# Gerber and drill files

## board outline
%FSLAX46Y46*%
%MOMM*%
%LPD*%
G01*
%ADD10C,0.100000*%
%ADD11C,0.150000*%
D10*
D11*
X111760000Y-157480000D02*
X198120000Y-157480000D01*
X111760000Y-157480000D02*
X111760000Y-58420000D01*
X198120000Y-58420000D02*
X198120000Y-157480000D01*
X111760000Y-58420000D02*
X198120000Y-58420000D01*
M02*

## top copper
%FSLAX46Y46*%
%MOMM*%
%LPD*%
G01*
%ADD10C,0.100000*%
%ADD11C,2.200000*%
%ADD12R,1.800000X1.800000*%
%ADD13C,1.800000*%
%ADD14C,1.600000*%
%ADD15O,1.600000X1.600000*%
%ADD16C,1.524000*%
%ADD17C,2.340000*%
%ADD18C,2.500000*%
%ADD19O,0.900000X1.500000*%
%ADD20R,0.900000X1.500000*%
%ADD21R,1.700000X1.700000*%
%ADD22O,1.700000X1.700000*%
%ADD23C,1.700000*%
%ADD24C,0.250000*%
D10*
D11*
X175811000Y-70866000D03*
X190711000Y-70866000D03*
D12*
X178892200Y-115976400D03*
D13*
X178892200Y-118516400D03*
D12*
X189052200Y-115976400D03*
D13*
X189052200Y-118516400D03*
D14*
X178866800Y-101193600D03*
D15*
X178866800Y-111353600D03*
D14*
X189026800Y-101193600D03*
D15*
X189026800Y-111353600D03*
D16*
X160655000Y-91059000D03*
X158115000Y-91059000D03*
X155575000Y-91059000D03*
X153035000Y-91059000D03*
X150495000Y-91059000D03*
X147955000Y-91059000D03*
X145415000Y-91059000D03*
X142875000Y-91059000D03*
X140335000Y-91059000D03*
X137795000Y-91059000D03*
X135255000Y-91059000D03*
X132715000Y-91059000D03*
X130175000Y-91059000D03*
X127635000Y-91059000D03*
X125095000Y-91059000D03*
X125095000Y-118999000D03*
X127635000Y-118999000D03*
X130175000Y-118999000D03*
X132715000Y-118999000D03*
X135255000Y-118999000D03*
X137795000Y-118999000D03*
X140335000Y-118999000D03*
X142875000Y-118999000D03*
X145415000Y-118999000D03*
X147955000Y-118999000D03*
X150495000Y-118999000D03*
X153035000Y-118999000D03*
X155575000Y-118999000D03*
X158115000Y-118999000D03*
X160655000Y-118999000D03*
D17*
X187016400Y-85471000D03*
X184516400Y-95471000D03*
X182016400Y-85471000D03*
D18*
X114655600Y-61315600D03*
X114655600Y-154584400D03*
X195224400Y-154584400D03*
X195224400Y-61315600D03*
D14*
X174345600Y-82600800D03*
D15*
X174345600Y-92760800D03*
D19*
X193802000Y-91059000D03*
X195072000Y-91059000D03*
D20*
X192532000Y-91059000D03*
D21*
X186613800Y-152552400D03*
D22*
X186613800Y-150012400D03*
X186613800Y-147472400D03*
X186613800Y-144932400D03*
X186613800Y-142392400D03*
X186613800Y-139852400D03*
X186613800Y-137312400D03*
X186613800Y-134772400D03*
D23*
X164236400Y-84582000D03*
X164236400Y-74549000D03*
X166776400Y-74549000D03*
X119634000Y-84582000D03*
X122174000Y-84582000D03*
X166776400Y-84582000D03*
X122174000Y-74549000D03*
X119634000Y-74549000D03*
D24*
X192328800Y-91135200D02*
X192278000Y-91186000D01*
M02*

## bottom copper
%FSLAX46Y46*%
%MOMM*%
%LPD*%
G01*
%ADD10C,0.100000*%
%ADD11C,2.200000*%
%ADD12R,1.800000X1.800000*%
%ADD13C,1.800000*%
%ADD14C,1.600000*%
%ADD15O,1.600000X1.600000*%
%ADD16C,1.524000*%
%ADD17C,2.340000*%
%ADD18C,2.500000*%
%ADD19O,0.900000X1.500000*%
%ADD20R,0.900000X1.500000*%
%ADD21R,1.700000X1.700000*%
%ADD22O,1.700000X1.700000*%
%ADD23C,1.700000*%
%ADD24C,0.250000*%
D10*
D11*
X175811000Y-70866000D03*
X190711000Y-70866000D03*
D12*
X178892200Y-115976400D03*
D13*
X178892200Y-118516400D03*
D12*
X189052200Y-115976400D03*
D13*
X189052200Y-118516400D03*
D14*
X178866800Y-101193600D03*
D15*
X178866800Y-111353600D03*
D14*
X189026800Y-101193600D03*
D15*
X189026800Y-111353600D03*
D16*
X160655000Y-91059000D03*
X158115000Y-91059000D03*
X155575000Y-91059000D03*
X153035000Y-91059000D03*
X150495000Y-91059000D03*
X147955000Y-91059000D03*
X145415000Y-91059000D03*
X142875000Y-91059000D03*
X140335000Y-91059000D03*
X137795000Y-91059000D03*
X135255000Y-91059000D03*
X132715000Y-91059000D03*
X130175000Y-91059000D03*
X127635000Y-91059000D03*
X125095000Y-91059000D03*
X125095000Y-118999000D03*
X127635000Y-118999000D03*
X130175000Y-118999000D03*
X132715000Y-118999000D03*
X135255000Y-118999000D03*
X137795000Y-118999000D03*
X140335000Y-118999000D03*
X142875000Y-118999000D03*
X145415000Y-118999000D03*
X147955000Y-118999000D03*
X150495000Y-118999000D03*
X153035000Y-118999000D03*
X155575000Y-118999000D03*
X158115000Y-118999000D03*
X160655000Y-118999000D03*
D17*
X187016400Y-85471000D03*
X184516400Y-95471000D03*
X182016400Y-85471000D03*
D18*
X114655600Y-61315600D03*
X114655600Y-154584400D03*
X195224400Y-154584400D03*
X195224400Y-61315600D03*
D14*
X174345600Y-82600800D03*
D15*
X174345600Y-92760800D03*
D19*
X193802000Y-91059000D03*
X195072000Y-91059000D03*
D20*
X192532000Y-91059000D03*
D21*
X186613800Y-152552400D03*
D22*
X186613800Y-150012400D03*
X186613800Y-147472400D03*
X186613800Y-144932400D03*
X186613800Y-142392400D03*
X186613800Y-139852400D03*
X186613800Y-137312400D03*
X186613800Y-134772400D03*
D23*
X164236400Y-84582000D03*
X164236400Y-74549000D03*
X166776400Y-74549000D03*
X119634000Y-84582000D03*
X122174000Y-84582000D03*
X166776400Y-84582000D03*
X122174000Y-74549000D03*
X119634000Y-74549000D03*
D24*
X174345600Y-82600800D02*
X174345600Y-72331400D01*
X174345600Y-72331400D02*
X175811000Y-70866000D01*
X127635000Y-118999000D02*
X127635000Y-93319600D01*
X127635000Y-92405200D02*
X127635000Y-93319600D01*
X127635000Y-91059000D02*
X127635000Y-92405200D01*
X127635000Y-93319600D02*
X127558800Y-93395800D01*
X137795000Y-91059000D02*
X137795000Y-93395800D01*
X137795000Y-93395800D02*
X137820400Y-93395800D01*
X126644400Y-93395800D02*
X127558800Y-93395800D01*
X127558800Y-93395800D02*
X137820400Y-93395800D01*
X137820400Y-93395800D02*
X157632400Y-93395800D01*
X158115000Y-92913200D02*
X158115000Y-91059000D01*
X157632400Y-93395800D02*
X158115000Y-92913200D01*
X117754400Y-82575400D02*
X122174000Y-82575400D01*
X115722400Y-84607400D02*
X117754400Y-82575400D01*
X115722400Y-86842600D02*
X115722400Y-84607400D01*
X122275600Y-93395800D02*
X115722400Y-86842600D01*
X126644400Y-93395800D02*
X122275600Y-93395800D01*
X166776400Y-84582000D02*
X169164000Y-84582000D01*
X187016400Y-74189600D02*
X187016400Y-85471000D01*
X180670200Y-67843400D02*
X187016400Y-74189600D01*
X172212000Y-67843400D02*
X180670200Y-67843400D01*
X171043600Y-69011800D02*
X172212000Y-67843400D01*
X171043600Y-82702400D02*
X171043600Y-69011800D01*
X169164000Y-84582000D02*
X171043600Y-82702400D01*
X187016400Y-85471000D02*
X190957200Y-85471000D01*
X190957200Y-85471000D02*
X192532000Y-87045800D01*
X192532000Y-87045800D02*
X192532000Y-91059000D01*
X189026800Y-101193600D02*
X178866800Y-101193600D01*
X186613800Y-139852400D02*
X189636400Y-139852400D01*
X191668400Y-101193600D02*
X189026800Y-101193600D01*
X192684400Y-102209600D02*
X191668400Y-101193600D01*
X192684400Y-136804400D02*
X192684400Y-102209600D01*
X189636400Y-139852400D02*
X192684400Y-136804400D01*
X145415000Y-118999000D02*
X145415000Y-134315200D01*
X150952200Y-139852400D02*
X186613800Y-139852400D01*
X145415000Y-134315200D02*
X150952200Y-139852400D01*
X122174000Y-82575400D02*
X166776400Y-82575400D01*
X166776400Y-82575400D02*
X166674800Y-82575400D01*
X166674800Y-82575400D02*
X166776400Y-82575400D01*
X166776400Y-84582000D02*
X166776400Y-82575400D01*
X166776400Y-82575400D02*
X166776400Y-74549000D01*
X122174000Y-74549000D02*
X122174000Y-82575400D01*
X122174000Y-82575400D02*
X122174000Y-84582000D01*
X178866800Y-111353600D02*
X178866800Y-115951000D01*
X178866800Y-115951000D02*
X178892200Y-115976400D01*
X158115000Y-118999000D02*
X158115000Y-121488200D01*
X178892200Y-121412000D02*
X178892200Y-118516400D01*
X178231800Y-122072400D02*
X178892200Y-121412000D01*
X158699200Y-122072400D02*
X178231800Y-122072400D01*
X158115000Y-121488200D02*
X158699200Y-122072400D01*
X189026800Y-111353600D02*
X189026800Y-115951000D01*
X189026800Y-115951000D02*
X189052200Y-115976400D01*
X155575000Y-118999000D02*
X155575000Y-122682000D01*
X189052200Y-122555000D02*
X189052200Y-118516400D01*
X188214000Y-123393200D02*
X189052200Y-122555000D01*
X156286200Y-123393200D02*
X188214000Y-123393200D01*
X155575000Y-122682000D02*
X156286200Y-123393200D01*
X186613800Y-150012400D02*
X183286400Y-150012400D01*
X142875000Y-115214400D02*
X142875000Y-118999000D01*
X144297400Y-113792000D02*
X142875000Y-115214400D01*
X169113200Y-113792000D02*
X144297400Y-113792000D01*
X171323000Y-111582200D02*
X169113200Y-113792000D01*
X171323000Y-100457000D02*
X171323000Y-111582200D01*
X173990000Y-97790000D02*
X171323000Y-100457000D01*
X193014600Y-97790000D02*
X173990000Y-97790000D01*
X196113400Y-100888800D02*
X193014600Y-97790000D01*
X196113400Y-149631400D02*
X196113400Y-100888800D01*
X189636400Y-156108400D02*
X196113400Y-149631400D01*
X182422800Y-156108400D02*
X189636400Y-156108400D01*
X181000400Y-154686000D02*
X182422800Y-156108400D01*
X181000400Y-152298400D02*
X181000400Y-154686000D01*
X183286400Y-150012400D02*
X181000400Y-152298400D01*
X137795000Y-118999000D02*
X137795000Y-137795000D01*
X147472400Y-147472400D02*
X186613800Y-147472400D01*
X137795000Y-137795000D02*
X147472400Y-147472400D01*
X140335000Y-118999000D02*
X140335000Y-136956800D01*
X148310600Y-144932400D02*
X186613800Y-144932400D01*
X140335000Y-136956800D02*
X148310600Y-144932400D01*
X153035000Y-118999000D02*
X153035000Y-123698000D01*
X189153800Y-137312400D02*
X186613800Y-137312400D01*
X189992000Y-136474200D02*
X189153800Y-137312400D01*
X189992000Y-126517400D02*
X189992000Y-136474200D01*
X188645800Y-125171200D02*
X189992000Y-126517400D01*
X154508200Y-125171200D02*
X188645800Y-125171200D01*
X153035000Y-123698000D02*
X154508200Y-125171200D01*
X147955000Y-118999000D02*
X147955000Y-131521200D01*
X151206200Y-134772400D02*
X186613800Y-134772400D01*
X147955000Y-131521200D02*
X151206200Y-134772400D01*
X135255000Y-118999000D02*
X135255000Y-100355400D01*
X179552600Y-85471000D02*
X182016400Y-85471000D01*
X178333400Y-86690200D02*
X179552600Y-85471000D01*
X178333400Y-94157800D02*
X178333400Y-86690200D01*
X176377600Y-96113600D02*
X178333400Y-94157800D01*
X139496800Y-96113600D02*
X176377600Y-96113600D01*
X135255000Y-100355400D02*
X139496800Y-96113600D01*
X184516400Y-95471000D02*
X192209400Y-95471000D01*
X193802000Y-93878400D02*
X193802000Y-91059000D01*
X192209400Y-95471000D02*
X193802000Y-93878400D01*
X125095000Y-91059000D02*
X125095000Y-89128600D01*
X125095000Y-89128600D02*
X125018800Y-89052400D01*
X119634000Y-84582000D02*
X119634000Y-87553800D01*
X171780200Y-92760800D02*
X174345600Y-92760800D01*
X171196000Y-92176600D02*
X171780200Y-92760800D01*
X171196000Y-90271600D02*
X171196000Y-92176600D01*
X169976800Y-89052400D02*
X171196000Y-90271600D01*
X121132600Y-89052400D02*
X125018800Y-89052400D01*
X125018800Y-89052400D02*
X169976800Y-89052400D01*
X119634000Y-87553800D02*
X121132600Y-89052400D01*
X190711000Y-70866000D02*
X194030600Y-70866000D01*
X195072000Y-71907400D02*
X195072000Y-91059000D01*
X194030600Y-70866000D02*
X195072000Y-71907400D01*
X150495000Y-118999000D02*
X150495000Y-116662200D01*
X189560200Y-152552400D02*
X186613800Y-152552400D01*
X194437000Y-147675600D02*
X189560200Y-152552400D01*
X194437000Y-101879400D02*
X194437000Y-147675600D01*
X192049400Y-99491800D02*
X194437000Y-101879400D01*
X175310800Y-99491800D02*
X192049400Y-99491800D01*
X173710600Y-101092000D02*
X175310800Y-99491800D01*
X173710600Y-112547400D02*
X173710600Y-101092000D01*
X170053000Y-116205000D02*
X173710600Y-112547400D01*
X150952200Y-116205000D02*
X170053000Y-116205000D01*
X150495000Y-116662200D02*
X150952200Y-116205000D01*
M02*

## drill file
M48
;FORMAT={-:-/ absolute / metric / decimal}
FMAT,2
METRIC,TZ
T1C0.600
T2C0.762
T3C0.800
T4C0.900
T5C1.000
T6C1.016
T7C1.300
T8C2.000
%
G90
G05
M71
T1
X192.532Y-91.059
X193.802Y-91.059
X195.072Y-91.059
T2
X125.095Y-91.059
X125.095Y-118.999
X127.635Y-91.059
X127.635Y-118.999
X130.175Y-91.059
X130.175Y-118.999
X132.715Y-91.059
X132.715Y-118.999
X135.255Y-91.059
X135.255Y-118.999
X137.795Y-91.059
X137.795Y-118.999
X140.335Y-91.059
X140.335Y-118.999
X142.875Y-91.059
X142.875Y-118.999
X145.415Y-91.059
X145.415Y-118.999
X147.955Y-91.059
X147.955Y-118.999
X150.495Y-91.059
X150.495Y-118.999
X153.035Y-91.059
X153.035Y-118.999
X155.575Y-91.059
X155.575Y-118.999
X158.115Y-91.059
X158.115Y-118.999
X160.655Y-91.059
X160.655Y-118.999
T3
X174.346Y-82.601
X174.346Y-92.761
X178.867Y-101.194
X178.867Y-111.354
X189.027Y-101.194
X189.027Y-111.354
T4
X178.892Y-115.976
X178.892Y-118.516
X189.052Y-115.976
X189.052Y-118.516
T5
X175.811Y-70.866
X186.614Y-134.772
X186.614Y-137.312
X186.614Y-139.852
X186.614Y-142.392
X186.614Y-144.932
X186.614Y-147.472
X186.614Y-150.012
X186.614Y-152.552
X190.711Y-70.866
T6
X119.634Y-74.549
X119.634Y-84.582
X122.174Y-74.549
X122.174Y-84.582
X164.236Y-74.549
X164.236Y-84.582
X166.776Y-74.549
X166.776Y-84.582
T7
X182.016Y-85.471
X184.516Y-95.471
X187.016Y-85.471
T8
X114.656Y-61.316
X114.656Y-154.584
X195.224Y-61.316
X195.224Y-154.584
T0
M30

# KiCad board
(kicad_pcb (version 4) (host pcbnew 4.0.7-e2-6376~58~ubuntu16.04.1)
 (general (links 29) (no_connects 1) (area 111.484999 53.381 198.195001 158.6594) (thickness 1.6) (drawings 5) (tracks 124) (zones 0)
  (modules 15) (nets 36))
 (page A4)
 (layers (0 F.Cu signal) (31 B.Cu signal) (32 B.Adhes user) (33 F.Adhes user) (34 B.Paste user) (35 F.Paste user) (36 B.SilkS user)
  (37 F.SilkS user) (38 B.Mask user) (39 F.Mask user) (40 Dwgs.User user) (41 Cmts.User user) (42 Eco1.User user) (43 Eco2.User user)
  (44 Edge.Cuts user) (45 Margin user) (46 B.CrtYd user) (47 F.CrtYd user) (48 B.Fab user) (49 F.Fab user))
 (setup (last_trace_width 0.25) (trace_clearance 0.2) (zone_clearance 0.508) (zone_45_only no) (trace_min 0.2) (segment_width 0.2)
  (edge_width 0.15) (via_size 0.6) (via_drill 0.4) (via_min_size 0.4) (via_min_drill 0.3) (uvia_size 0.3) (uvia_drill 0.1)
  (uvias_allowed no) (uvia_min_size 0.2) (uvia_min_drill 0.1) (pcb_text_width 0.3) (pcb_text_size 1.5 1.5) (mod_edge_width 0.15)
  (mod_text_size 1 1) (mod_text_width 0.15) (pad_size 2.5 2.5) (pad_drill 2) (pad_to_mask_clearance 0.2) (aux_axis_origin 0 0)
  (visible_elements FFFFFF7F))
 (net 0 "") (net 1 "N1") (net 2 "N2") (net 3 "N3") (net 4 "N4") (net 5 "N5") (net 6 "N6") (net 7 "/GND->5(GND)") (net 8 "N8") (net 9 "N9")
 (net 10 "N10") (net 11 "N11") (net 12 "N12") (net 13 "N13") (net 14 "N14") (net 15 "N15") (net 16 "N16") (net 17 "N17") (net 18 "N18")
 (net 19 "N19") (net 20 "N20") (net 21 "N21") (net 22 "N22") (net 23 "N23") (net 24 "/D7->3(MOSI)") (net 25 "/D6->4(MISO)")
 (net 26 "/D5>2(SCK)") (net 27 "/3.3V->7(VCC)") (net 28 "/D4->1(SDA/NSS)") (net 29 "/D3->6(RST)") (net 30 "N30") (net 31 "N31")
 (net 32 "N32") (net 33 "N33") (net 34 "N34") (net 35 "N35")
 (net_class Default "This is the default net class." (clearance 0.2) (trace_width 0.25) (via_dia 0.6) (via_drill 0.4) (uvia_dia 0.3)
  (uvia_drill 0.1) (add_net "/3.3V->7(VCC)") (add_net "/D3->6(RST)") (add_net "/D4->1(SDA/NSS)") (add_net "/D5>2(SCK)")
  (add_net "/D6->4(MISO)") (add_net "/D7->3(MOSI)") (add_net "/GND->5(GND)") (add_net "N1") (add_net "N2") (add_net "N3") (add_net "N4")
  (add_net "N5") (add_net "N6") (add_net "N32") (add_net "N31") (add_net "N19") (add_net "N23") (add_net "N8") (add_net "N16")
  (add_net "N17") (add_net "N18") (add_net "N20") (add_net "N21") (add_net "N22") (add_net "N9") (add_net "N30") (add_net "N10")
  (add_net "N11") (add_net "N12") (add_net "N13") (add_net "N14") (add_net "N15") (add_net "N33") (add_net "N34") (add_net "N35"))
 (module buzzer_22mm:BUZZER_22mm (layer F.Cu) (at 183.261 70.866)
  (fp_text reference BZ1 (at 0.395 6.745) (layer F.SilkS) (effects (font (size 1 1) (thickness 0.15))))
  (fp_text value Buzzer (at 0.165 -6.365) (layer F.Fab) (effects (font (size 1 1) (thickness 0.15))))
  (pad 1 thru_hole circle (at -7.45 0) (size 2.2 2.2) (drill 1) (layers *.Cu *.Mask) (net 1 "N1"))
  (pad 2 thru_hole circle (at 7.45 0) (size 2.2 2.2) (drill 1) (layers *.Cu *.Mask) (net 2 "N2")))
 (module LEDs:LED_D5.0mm (layer F.Cu) (at 178.8922 115.9764 270)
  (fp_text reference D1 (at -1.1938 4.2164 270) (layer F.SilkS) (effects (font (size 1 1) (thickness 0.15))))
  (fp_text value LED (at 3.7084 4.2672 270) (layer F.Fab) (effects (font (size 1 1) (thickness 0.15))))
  (pad 1 thru_hole rect (at 0 0 270) (size 1.8 1.8) (drill 0.9) (layers *.Cu *.Mask) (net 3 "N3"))
  (pad 2 thru_hole circle (at 2.54 0 270) (size 1.8 1.8) (drill 0.9) (layers *.Cu *.Mask) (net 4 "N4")))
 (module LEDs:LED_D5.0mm (layer F.Cu) (at 189.0522 115.9764 270)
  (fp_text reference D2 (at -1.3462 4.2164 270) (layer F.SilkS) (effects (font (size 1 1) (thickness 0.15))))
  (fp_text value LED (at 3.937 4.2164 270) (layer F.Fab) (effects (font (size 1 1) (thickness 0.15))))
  (pad 1 thru_hole rect (at 0 0 270) (size 1.8 1.8) (drill 0.9) (layers *.Cu *.Mask) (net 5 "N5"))
  (pad 2 thru_hole circle (at 2.54 0 270) (size 1.8 1.8) (drill 0.9) (layers *.Cu *.Mask) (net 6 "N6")))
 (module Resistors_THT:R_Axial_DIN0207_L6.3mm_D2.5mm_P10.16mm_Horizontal (layer F.Cu) (at 178.8668 101.1936 270)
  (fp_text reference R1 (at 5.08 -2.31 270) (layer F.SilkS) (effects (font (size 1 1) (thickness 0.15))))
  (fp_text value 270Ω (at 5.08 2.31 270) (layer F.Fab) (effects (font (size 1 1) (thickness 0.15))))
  (pad 1 thru_hole circle (at 0 0 270) (size 1.6 1.6) (drill 0.8) (layers *.Cu *.Mask) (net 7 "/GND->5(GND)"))
  (pad 2 thru_hole oval (at 10.16 0 270) (size 1.6 1.6) (drill 0.8) (layers *.Cu *.Mask) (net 3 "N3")))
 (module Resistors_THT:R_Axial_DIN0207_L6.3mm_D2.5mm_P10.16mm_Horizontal (layer F.Cu) (at 189.0268 101.1936 270)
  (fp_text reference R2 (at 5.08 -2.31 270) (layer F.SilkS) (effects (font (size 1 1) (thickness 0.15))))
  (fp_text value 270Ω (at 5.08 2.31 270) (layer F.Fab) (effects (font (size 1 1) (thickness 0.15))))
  (pad 1 thru_hole circle (at 0 0 270) (size 1.6 1.6) (drill 0.8) (layers *.Cu *.Mask) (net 7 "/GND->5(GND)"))
  (pad 2 thru_hole oval (at 10.16 0 270) (size 1.6 1.6) (drill 0.8) (layers *.Cu *.Mask) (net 5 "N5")))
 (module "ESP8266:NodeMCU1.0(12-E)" (layer F.Cu) (at 139.7 105.029 270)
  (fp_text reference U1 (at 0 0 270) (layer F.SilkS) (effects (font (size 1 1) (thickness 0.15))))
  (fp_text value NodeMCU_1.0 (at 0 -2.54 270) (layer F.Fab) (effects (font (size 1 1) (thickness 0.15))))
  (pad 1 thru_hole circle (at -13.97 -20.955 270) (size 1.524 1.524) (drill 0.762) (layers *.Cu *.Mask F.SilkS) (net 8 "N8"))
  (pad 2 thru_hole circle (at -13.97 -18.415 270) (size 1.524 1.524) (drill 0.762) (layers *.Cu *.Mask F.SilkS) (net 7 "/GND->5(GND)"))
  (pad 3 thru_hole circle (at -13.97 -15.875 270) (size 1.524 1.524) (drill 0.762) (layers *.Cu *.Mask F.SilkS) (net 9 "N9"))
  (pad 4 thru_hole circle (at -13.97 -13.335 270) (size 1.524 1.524) (drill 0.762) (layers *.Cu *.Mask F.SilkS) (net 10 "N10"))
  (pad 5 thru_hole circle (at -13.97 -10.795 270) (size 1.524 1.524) (drill 0.762) (layers *.Cu *.Mask F.SilkS) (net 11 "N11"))
  (pad 6 thru_hole circle (at -13.97 -8.255 270) (size 1.524 1.524) (drill 0.762) (layers *.Cu *.Mask F.SilkS) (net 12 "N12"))
  (pad 7 thru_hole circle (at -13.97 -5.715 270) (size 1.524 1.524) (drill 0.762) (layers *.Cu *.Mask F.SilkS) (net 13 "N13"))
  (pad 8 thru_hole circle (at -13.97 -3.175 270) (size 1.524 1.524) (drill 0.762) (layers *.Cu *.Mask F.SilkS) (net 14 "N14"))
  (pad 9 thru_hole circle (at -13.97 -0.635 270) (size 1.524 1.524) (drill 0.762) (layers *.Cu *.Mask F.SilkS) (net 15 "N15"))
  (pad 10 thru_hole circle (at -13.97 1.905 270) (size 1.524 1.524) (drill 0.762) (layers *.Cu *.Mask F.SilkS) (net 7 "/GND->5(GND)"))
  (pad 11 thru_hole circle (at -13.97 4.445 270) (size 1.524 1.524) (drill 0.762) (layers *.Cu *.Mask F.SilkS) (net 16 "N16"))
  (pad 12 thru_hole circle (at -13.97 6.985 270) (size 1.524 1.524) (drill 0.762) (layers *.Cu *.Mask F.SilkS) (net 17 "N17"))
  (pad 13 thru_hole circle (at -13.97 9.525 270) (size 1.524 1.524) (drill 0.762) (layers *.Cu *.Mask F.SilkS) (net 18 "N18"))
  (pad 14 thru_hole circle (at -13.97 12.065 270) (size 1.524 1.524) (drill 0.762) (layers *.Cu *.Mask F.SilkS) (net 7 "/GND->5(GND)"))
  (pad 15 thru_hole circle (at -13.97 14.605 270) (size 1.524 1.524) (drill 0.762) (layers *.Cu *.Mask F.SilkS) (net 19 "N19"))
  (pad 16 thru_hole circle (at 13.97 14.605 270) (size 1.524 1.524) (drill 0.762) (layers *.Cu *.Mask F.SilkS) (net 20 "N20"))
  (pad 17 thru_hole circle (at 13.97 12.065 270) (size 1.524 1.524) (drill 0.762) (layers *.Cu *.Mask F.SilkS) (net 7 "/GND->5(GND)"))
  (pad 18 thru_hole circle (at 13.97 9.525 270) (size 1.524 1.524) (drill 0.762) (layers *.Cu *.Mask F.SilkS) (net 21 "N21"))
  (pad 19 thru_hole circle (at 13.97 6.985 270) (size 1.524 1.524) (drill 0.762) (layers *.Cu *.Mask F.SilkS) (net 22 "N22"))
  (pad 20 thru_hole circle (at 13.97 4.445 270) (size 1.524 1.524) (drill 0.762) (layers *.Cu *.Mask F.SilkS) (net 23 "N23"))
  (pad 21 thru_hole circle (at 13.97 1.905 270) (size 1.524 1.524) (drill 0.762) (layers *.Cu *.Mask F.SilkS) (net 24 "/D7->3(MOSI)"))
  (pad 22 thru_hole circle (at 13.97 -0.635 270) (size 1.524 1.524) (drill 0.762) (layers *.Cu *.Mask F.SilkS) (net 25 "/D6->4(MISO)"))
  (pad 23 thru_hole circle (at 13.97 -3.175 270) (size 1.524 1.524) (drill 0.762) (layers *.Cu *.Mask F.SilkS) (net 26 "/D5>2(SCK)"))
  (pad 24 thru_hole circle (at 13.97 -5.715 270) (size 1.524 1.524) (drill 0.762) (layers *.Cu *.Mask F.SilkS) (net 7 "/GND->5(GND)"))
  (pad 25 thru_hole circle (at 13.97 -8.255 270) (size 1.524 1.524) (drill 0.762) (layers *.Cu *.Mask F.SilkS) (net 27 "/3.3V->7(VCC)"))
  (pad 26 thru_hole circle (at 13.97 -10.795 270) (size 1.524 1.524) (drill 0.762) (layers *.Cu *.Mask F.SilkS) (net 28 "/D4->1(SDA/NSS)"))
  (pad 27 thru_hole circle (at 13.97 -13.335 270) (size 1.524 1.524) (drill 0.762) (layers *.Cu *.Mask F.SilkS) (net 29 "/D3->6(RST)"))
  (pad 28 thru_hole circle (at 13.97 -15.875 270) (size 1.524 1.524) (drill 0.762) (layers *.Cu *.Mask F.SilkS) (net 6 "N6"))
  (pad 29 thru_hole circle (at 13.97 -18.415 270) (size 1.524 1.524) (drill 0.762) (layers *.Cu *.Mask F.SilkS) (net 4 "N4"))
  (pad 30 thru_hole circle (at 13.97 -20.955 270) (size 1.524 1.524) (drill 0.762) (layers *.Cu *.Mask F.SilkS) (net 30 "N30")))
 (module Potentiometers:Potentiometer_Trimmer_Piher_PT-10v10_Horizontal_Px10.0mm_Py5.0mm (layer F.Cu) (at 182.0164 85.471 270)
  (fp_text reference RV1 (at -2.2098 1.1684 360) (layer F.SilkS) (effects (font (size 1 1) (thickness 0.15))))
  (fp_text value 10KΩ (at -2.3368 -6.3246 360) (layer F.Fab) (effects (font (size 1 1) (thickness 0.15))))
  (pad 3 thru_hole circle (at 0 -5 270) (size 2.34 2.34) (drill 1.3) (layers *.Cu *.Mask) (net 7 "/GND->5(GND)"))
  (pad 2 thru_hole circle (at 10 -2.5 270) (size 2.34 2.34) (drill 1.3) (layers *.Cu *.Mask) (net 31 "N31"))
  (pad 1 thru_hole circle (at 0 0 270) (size 2.34 2.34) (drill 1.3) (layers *.Cu *.Mask) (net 23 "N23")))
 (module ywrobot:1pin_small (layer F.Cu) (at 114.6556 61.3156)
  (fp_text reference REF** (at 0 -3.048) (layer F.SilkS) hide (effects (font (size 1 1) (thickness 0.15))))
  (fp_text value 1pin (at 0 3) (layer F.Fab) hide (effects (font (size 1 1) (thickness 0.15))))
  (pad 1 thru_hole circle (at 0 0) (size 2.5 2.5) (drill 2) (layers *.Cu *.Mask) (zone_connect 0)))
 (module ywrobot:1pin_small (layer F.Cu) (at 114.6556 154.5844)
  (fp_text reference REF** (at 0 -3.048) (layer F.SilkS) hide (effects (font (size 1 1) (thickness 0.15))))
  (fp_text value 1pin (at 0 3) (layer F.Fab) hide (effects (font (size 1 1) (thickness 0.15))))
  (pad 2 thru_hole circle (at 0 0) (size 2.5 2.5) (drill 2) (layers *.Cu *.Mask) (zone_connect 0)))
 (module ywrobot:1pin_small (layer F.Cu) (at 195.2244 154.5844)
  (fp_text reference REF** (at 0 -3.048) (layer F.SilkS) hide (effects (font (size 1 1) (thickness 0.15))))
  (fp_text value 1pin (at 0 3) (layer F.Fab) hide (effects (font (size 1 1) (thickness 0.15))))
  (pad 3 thru_hole circle (at 0 0) (size 2.5 2.5) (drill 2) (layers *.Cu *.Mask) (zone_connect 0)))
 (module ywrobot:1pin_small (layer F.Cu) (at 195.2244 61.3156)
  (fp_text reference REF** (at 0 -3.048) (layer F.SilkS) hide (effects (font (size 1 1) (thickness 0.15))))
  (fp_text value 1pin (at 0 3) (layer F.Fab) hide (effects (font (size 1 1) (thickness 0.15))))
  (pad 4 thru_hole circle (at 0 0) (size 2.5 2.5) (drill 2) (layers *.Cu *.Mask) (zone_connect 0)))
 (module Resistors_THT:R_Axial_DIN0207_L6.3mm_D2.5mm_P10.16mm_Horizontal (layer F.Cu) (at 174.3456 82.6008 270)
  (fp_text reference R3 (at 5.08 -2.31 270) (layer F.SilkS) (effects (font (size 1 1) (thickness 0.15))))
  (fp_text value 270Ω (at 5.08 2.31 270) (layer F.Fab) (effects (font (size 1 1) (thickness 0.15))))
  (pad 1 thru_hole circle (at 0 0 270) (size 1.6 1.6) (drill 0.8) (layers *.Cu *.Mask) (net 1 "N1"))
  (pad 2 thru_hole oval (at 10.16 0 270) (size 1.6 1.6) (drill 0.8) (layers *.Cu *.Mask) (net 19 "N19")))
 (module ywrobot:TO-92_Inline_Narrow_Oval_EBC (layer F.Cu) (at 192.532 91.059)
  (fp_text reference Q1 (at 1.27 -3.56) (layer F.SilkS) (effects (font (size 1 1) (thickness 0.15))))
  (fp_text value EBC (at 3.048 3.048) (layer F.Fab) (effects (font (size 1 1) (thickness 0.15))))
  (pad 1 thru_hole oval (at 1.27 0 180) (size 0.9 1.5) (drill 0.6) (layers *.Cu *.Mask) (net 31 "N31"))
  (pad 2 thru_hole oval (at 2.54 0 180) (size 0.9 1.5) (drill 0.6) (layers *.Cu *.Mask) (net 2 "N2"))
  (pad 3 thru_hole rect (at 0 0 180) (size 0.9 1.5) (drill 0.6) (layers *.Cu *.Mask) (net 7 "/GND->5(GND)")))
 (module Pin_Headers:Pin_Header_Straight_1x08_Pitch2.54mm (layer F.Cu) (at 186.6138 152.5524 180)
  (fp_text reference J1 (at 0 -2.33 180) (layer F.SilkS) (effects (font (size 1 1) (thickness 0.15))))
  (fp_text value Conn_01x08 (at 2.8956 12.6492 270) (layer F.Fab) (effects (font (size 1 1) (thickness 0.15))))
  (pad 1 thru_hole rect (at 0 0 180) (size 1.7 1.7) (drill 1) (layers *.Cu *.Mask) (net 28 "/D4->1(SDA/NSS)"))
  (pad 2 thru_hole oval (at 0 2.54 180) (size 1.7 1.7) (drill 1) (layers *.Cu *.Mask) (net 26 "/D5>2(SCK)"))
  (pad 3 thru_hole oval (at 0 5.08 180) (size 1.7 1.7) (drill 1) (layers *.Cu *.Mask) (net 24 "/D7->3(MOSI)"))
  (pad 4 thru_hole oval (at 0 7.62 180) (size 1.7 1.7) (drill 1) (layers *.Cu *.Mask) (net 25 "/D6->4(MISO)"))
  (pad 5 thru_hole oval (at 0 10.16 180) (size 1.7 1.7) (drill 1) (layers *.Cu *.Mask) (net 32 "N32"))
  (pad 6 thru_hole oval (at 0 12.7 180) (size 1.7 1.7) (drill 1) (layers *.Cu *.Mask) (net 7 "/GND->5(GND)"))
  (pad 7 thru_hole oval (at 0 15.24 180) (size 1.7 1.7) (drill 1) (layers *.Cu *.Mask) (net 29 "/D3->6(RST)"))
  (pad 8 thru_hole oval (at 0 17.78 180) (size 1.7 1.7) (drill 1) (layers *.Cu *.Mask) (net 27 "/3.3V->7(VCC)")))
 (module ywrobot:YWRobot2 (layer F.Cu) (at 143.002 56.896 180)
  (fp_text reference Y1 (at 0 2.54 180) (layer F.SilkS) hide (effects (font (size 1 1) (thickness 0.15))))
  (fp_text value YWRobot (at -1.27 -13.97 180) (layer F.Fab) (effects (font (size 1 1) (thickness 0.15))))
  (pad 1 thru_hole circle (at -21.2344 -27.686 180) (size 1.7 1.7) (drill 1.016) (layers *.Cu *.Mask) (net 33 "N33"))
  (pad 2 thru_hole circle (at -21.2344 -17.653 180) (size 1.7 1.7) (drill 1.016) (layers *.Cu *.Mask) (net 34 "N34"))
  (pad 3 thru_hole circle (at -23.7744 -17.653 180) (size 1.7 1.7) (drill 1.016) (layers *.Cu *.Mask) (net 7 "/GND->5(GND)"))
  (pad 4 thru_hole circle (at 23.368 -27.686 180) (size 1.7 1.7) (drill 1.016) (layers *.Cu *.Mask) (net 19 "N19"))
  (pad 5 thru_hole circle (at 20.828 -27.686 180) (size 1.7 1.7) (drill 1.016) (layers *.Cu *.Mask) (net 7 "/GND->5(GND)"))
  (pad 6 thru_hole circle (at -23.7744 -27.686 180) (size 1.7 1.7) (drill 1.016) (layers *.Cu *.Mask) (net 7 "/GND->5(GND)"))
  (pad 7 thru_hole circle (at 20.828 -17.653 180) (size 1.7 1.7) (drill 1.016) (layers *.Cu *.Mask) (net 7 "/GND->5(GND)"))
  (pad 8 thru_hole circle (at 23.368 -17.653 180) (size 1.7 1.7) (drill 1.016) (layers *.Cu *.Mask) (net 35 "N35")))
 (gr_line (start 111.76 157.48) (end 198.12 157.48) (angle 90) (layer Edge.Cuts) (width 0.15))
 (gr_line (start 111.76 157.48) (end 111.76 58.42) (angle 90) (layer Edge.Cuts) (width 0.15))
 (gr_line (start 198.12 58.42) (end 198.12 157.48) (angle 90) (layer Edge.Cuts) (width 0.15))
 (gr_line (start 111.76 58.42) (end 198.12 58.42) (angle 90) (layer Edge.Cuts) (width 0.15))
 (segment (start 174.3456 82.6008) (end 174.3456 72.3314) (width 0.25) (layer B.Cu) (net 1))
 (segment (start 174.3456 72.3314) (end 175.811 70.866) (width 0.25) (layer B.Cu) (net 1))
 (segment (start 127.635 118.999) (end 127.635 93.3196) (width 0.25) (layer B.Cu) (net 7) (status 400000))
 (segment (start 127.635 92.4052) (end 127.635 93.3196) (width 0.25) (layer B.Cu) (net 7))
 (segment (start 127.635 91.059) (end 127.635 92.4052) (width 0.25) (layer B.Cu) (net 7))
 (segment (start 127.635 93.3196) (end 127.5588 93.3958) (width 0.25) (layer B.Cu) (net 7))
 (segment (start 137.795 91.059) (end 137.795 93.3958) (width 0.25) (layer B.Cu) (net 7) (status 400000))
 (segment (start 137.795 93.3958) (end 137.8204 93.3958) (width 0.25) (layer B.Cu) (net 7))
 (segment (start 126.6444 93.3958) (end 127.5588 93.3958) (width 0.25) (layer B.Cu) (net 7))
 (segment (start 127.5588 93.3958) (end 137.8204 93.3958) (width 0.25) (layer B.Cu) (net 7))
 (segment (start 137.8204 93.3958) (end 157.6324 93.3958) (width 0.25) (layer B.Cu) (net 7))
 (segment (start 158.115 92.9132) (end 158.115 91.059) (width 0.25) (layer B.Cu) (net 7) (status 800000))
 (segment (start 157.6324 93.3958) (end 158.115 92.9132) (width 0.25) (layer B.Cu) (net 7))
 (segment (start 117.7544 82.5754) (end 122.174 82.5754) (width 0.25) (layer B.Cu) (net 7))
 (segment (start 115.7224 84.6074) (end 117.7544 82.5754) (width 0.25) (layer B.Cu) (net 7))
 (segment (start 115.7224 86.8426) (end 115.7224 84.6074) (width 0.25) (layer B.Cu) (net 7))
 (segment (start 122.2756 93.3958) (end 115.7224 86.8426) (width 0.25) (layer B.Cu) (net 7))
 (segment (start 126.6444 93.3958) (end 122.2756 93.3958) (width 0.25) (layer B.Cu) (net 7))
 (segment (start 166.7764 84.582) (end 169.164 84.582) (width 0.25) (layer B.Cu) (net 7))
 (segment (start 187.0164 74.1896) (end 187.0164 85.471) (width 0.25) (layer B.Cu) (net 7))
 (segment (start 180.6702 67.8434) (end 187.0164 74.1896) (width 0.25) (layer B.Cu) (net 7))
 (segment (start 172.212 67.8434) (end 180.6702 67.8434) (width 0.25) (layer B.Cu) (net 7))
 (segment (start 171.0436 69.0118) (end 172.212 67.8434) (width 0.25) (layer B.Cu) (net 7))
 (segment (start 171.0436 82.7024) (end 171.0436 69.0118) (width 0.25) (layer B.Cu) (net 7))
 (segment (start 169.164 84.582) (end 171.0436 82.7024) (width 0.25) (layer B.Cu) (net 7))
 (segment (start 187.0164 85.471) (end 190.9572 85.471) (width 0.25) (layer B.Cu) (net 7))
 (segment (start 190.9572 85.471) (end 192.532 87.0458) (width 0.25) (layer B.Cu) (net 7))
 (segment (start 192.532 87.0458) (end 192.532 91.059) (width 0.25) (layer B.Cu) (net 7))
 (segment (start 189.0268 101.1936) (end 178.8668 101.1936) (width 0.25) (layer B.Cu) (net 7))
 (segment (start 186.6138 139.8524) (end 189.6364 139.8524) (width 0.25) (layer B.Cu) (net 7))
 (segment (start 191.6684 101.1936) (end 189.0268 101.1936) (width 0.25) (layer B.Cu) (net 7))
 (segment (start 192.6844 102.2096) (end 191.6684 101.1936) (width 0.25) (layer B.Cu) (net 7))
 (segment (start 192.6844 136.8044) (end 192.6844 102.2096) (width 0.25) (layer B.Cu) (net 7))
 (segment (start 189.6364 139.8524) (end 192.6844 136.8044) (width 0.25) (layer B.Cu) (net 7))
 (segment (start 145.415 118.999) (end 145.415 134.3152) (width 0.25) (layer B.Cu) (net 7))
 (segment (start 150.9522 139.8524) (end 186.6138 139.8524) (width 0.25) (layer B.Cu) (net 7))
 (segment (start 145.415 134.3152) (end 150.9522 139.8524) (width 0.25) (layer B.Cu) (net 7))
 (segment (start 122.174 82.5754) (end 166.7764 82.5754) (width 0.25) (layer B.Cu) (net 7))
 (segment (start 166.7764 82.5754) (end 166.6748 82.5754) (width 0.25) (layer B.Cu) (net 7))
 (segment (start 166.6748 82.5754) (end 166.7764 82.5754) (width 0.25) (layer B.Cu) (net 7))
 (segment (start 166.7764 84.582) (end 166.7764 82.5754) (width 0.25) (layer B.Cu) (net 7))
 (segment (start 166.7764 82.5754) (end 166.7764 74.549) (width 0.25) (layer B.Cu) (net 7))
 (segment (start 122.174 74.549) (end 122.174 82.5754) (width 0.25) (layer B.Cu) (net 7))
 (segment (start 122.174 82.5754) (end 122.174 84.582) (width 0.25) (layer B.Cu) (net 7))
 (segment (start 192.3288 91.1352) (end 192.278 91.186) (width 0.25) (layer F.Cu) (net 7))
 (segment (start 178.8668 111.3536) (end 178.8668 115.951) (width 0.25) (layer B.Cu) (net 3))
 (segment (start 178.8668 115.951) (end 178.8922 115.9764) (width 0.25) (layer B.Cu) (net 3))
 (segment (start 158.115 118.999) (end 158.115 121.4882) (width 0.25) (layer B.Cu) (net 4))
 (segment (start 178.8922 121.412) (end 178.8922 118.5164) (width 0.25) (layer B.Cu) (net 4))
 (segment (start 178.2318 122.0724) (end 178.8922 121.412) (width 0.25) (layer B.Cu) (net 4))
 (segment (start 158.6992 122.0724) (end 178.2318 122.0724) (width 0.25) (layer B.Cu) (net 4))
 (segment (start 158.115 121.4882) (end 158.6992 122.0724) (width 0.25) (layer B.Cu) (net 4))
 (segment (start 189.0268 111.3536) (end 189.0268 115.951) (width 0.25) (layer B.Cu) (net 5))
 (segment (start 189.0268 115.951) (end 189.0522 115.9764) (width 0.25) (layer B.Cu) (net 5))
 (segment (start 155.575 118.999) (end 155.575 122.682) (width 0.25) (layer B.Cu) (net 6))
 (segment (start 189.0522 122.555) (end 189.0522 118.5164) (width 0.25) (layer B.Cu) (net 6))
 (segment (start 188.214 123.3932) (end 189.0522 122.555) (width 0.25) (layer B.Cu) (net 6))
 (segment (start 156.2862 123.3932) (end 188.214 123.3932) (width 0.25) (layer B.Cu) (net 6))
 (segment (start 155.575 122.682) (end 156.2862 123.3932) (width 0.25) (layer B.Cu) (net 6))
 (segment (start 186.6138 150.0124) (end 183.2864 150.0124) (width 0.25) (layer B.Cu) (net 26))
 (segment (start 142.875 115.2144) (end 142.875 118.999) (width 0.25) (layer B.Cu) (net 26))
 (segment (start 144.2974 113.792) (end 142.875 115.2144) (width 0.25) (layer B.Cu) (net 26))
 (segment (start 169.1132 113.792) (end 144.2974 113.792) (width 0.25) (layer B.Cu) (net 26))
 (segment (start 171.323 111.5822) (end 169.1132 113.792) (width 0.25) (layer B.Cu) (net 26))
 (segment (start 171.323 100.457) (end 171.323 111.5822) (width 0.25) (layer B.Cu) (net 26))
 (segment (start 173.99 97.79) (end 171.323 100.457) (width 0.25) (layer B.Cu) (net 26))
 (segment (start 193.0146 97.79) (end 173.99 97.79) (width 0.25) (layer B.Cu) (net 26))
 (segment (start 196.1134 100.8888) (end 193.0146 97.79) (width 0.25) (layer B.Cu) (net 26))
 (segment (start 196.1134 149.6314) (end 196.1134 100.8888) (width 0.25) (layer B.Cu) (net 26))
 (segment (start 189.6364 156.1084) (end 196.1134 149.6314) (width 0.25) (layer B.Cu) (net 26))
 (segment (start 182.4228 156.1084) (end 189.6364 156.1084) (width 0.25) (layer B.Cu) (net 26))
 (segment (start 181.0004 154.686) (end 182.4228 156.1084) (width 0.25) (layer B.Cu) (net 26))
 (segment (start 181.0004 152.2984) (end 181.0004 154.686) (width 0.25) (layer B.Cu) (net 26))
 (segment (start 183.2864 150.0124) (end 181.0004 152.2984) (width 0.25) (layer B.Cu) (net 26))
 (segment (start 137.795 118.999) (end 137.795 137.795) (width 0.25) (layer B.Cu) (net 24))
 (segment (start 147.4724 147.4724) (end 186.6138 147.4724) (width 0.25) (layer B.Cu) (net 24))
 (segment (start 137.795 137.795) (end 147.4724 147.4724) (width 0.25) (layer B.Cu) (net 24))
 (segment (start 140.335 118.999) (end 140.335 136.9568) (width 0.25) (layer B.Cu) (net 25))
 (segment (start 148.3106 144.9324) (end 186.6138 144.9324) (width 0.25) (layer B.Cu) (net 25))
 (segment (start 140.335 136.9568) (end 148.3106 144.9324) (width 0.25) (layer B.Cu) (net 25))
 (segment (start 153.035 118.999) (end 153.035 123.698) (width 0.25) (layer B.Cu) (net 29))
 (segment (start 189.1538 137.3124) (end 186.6138 137.3124) (width 0.25) (layer B.Cu) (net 29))
 (segment (start 189.992 136.4742) (end 189.1538 137.3124) (width 0.25) (layer B.Cu) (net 29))
 (segment (start 189.992 126.5174) (end 189.992 136.4742) (width 0.25) (layer B.Cu) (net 29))
 (segment (start 188.6458 125.1712) (end 189.992 126.5174) (width 0.25) (layer B.Cu) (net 29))
 (segment (start 154.5082 125.1712) (end 188.6458 125.1712) (width 0.25) (layer B.Cu) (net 29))
 (segment (start 153.035 123.698) (end 154.5082 125.1712) (width 0.25) (layer B.Cu) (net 29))
 (segment (start 147.955 118.999) (end 147.955 131.5212) (width 0.25) (layer B.Cu) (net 27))
 (segment (start 151.2062 134.7724) (end 186.6138 134.7724) (width 0.25) (layer B.Cu) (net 27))
 (segment (start 147.955 131.5212) (end 151.2062 134.7724) (width 0.25) (layer B.Cu) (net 27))
 (segment (start 135.255 118.999) (end 135.255 100.3554) (width 0.25) (layer B.Cu) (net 23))
 (segment (start 179.5526 85.471) (end 182.0164 85.471) (width 0.25) (layer B.Cu) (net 23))
 (segment (start 178.3334 86.6902) (end 179.5526 85.471) (width 0.25) (layer B.Cu) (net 23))
 (segment (start 178.3334 94.1578) (end 178.3334 86.6902) (width 0.25) (layer B.Cu) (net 23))
 (segment (start 176.3776 96.1136) (end 178.3334 94.1578) (width 0.25) (layer B.Cu) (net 23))
 (segment (start 139.4968 96.1136) (end 176.3776 96.1136) (width 0.25) (layer B.Cu) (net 23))
 (segment (start 135.255 100.3554) (end 139.4968 96.1136) (width 0.25) (layer B.Cu) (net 23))
 (segment (start 184.5164 95.471) (end 192.2094 95.471) (width 0.25) (layer B.Cu) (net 31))
 (segment (start 193.802 93.8784) (end 193.802 91.059) (width 0.25) (layer B.Cu) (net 31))
 (segment (start 192.2094 95.471) (end 193.802 93.8784) (width 0.25) (layer B.Cu) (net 31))
 (segment (start 125.095 91.059) (end 125.095 89.1286) (width 0.25) (layer B.Cu) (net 19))
 (segment (start 125.095 89.1286) (end 125.0188 89.0524) (width 0.25) (layer B.Cu) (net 19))
 (segment (start 119.634 84.582) (end 119.634 87.5538) (width 0.25) (layer B.Cu) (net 19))
 (segment (start 171.7802 92.7608) (end 174.3456 92.7608) (width 0.25) (layer B.Cu) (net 19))
 (segment (start 171.196 92.1766) (end 171.7802 92.7608) (width 0.25) (layer B.Cu) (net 19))
 (segment (start 171.196 90.2716) (end 171.196 92.1766) (width 0.25) (layer B.Cu) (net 19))
 (segment (start 169.9768 89.0524) (end 171.196 90.2716) (width 0.25) (layer B.Cu) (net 19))
 (segment (start 121.1326 89.0524) (end 125.0188 89.0524) (width 0.25) (layer B.Cu) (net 19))
 (segment (start 125.0188 89.0524) (end 169.9768 89.0524) (width 0.25) (layer B.Cu) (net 19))
 (segment (start 119.634 87.5538) (end 121.1326 89.0524) (width 0.25) (layer B.Cu) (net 19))
 (segment (start 190.711 70.866) (end 194.0306 70.866) (width 0.25) (layer B.Cu) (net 2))
 (segment (start 195.072 71.9074) (end 195.072 91.059) (width 0.25) (layer B.Cu) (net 2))
 (segment (start 194.0306 70.866) (end 195.072 71.9074) (width 0.25) (layer B.Cu) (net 2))
 (segment (start 150.495 118.999) (end 150.495 116.6622) (width 0.25) (layer B.Cu) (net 28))
 (segment (start 189.5602 152.5524) (end 186.6138 152.5524) (width 0.25) (layer B.Cu) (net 28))
 (segment (start 194.437 147.6756) (end 189.5602 152.5524) (width 0.25) (layer B.Cu) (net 28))
 (segment (start 194.437 101.8794) (end 194.437 147.6756) (width 0.25) (layer B.Cu) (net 28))
 (segment (start 192.0494 99.4918) (end 194.437 101.8794) (width 0.25) (layer B.Cu) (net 28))
 (segment (start 175.3108 99.4918) (end 192.0494 99.4918) (width 0.25) (layer B.Cu) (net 28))
 (segment (start 173.7106 101.092) (end 175.3108 99.4918) (width 0.25) (layer B.Cu) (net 28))
 (segment (start 173.7106 112.5474) (end 173.7106 101.092) (width 0.25) (layer B.Cu) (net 28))
 (segment (start 170.053 116.205) (end 173.7106 112.5474) (width 0.25) (layer B.Cu) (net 28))
 (segment (start 150.9522 116.205) (end 170.053 116.205) (width 0.25) (layer B.Cu) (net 28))
 (segment (start 150.495 116.6622) (end 150.9522 116.205) (width 0.25) (layer B.Cu) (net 28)))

